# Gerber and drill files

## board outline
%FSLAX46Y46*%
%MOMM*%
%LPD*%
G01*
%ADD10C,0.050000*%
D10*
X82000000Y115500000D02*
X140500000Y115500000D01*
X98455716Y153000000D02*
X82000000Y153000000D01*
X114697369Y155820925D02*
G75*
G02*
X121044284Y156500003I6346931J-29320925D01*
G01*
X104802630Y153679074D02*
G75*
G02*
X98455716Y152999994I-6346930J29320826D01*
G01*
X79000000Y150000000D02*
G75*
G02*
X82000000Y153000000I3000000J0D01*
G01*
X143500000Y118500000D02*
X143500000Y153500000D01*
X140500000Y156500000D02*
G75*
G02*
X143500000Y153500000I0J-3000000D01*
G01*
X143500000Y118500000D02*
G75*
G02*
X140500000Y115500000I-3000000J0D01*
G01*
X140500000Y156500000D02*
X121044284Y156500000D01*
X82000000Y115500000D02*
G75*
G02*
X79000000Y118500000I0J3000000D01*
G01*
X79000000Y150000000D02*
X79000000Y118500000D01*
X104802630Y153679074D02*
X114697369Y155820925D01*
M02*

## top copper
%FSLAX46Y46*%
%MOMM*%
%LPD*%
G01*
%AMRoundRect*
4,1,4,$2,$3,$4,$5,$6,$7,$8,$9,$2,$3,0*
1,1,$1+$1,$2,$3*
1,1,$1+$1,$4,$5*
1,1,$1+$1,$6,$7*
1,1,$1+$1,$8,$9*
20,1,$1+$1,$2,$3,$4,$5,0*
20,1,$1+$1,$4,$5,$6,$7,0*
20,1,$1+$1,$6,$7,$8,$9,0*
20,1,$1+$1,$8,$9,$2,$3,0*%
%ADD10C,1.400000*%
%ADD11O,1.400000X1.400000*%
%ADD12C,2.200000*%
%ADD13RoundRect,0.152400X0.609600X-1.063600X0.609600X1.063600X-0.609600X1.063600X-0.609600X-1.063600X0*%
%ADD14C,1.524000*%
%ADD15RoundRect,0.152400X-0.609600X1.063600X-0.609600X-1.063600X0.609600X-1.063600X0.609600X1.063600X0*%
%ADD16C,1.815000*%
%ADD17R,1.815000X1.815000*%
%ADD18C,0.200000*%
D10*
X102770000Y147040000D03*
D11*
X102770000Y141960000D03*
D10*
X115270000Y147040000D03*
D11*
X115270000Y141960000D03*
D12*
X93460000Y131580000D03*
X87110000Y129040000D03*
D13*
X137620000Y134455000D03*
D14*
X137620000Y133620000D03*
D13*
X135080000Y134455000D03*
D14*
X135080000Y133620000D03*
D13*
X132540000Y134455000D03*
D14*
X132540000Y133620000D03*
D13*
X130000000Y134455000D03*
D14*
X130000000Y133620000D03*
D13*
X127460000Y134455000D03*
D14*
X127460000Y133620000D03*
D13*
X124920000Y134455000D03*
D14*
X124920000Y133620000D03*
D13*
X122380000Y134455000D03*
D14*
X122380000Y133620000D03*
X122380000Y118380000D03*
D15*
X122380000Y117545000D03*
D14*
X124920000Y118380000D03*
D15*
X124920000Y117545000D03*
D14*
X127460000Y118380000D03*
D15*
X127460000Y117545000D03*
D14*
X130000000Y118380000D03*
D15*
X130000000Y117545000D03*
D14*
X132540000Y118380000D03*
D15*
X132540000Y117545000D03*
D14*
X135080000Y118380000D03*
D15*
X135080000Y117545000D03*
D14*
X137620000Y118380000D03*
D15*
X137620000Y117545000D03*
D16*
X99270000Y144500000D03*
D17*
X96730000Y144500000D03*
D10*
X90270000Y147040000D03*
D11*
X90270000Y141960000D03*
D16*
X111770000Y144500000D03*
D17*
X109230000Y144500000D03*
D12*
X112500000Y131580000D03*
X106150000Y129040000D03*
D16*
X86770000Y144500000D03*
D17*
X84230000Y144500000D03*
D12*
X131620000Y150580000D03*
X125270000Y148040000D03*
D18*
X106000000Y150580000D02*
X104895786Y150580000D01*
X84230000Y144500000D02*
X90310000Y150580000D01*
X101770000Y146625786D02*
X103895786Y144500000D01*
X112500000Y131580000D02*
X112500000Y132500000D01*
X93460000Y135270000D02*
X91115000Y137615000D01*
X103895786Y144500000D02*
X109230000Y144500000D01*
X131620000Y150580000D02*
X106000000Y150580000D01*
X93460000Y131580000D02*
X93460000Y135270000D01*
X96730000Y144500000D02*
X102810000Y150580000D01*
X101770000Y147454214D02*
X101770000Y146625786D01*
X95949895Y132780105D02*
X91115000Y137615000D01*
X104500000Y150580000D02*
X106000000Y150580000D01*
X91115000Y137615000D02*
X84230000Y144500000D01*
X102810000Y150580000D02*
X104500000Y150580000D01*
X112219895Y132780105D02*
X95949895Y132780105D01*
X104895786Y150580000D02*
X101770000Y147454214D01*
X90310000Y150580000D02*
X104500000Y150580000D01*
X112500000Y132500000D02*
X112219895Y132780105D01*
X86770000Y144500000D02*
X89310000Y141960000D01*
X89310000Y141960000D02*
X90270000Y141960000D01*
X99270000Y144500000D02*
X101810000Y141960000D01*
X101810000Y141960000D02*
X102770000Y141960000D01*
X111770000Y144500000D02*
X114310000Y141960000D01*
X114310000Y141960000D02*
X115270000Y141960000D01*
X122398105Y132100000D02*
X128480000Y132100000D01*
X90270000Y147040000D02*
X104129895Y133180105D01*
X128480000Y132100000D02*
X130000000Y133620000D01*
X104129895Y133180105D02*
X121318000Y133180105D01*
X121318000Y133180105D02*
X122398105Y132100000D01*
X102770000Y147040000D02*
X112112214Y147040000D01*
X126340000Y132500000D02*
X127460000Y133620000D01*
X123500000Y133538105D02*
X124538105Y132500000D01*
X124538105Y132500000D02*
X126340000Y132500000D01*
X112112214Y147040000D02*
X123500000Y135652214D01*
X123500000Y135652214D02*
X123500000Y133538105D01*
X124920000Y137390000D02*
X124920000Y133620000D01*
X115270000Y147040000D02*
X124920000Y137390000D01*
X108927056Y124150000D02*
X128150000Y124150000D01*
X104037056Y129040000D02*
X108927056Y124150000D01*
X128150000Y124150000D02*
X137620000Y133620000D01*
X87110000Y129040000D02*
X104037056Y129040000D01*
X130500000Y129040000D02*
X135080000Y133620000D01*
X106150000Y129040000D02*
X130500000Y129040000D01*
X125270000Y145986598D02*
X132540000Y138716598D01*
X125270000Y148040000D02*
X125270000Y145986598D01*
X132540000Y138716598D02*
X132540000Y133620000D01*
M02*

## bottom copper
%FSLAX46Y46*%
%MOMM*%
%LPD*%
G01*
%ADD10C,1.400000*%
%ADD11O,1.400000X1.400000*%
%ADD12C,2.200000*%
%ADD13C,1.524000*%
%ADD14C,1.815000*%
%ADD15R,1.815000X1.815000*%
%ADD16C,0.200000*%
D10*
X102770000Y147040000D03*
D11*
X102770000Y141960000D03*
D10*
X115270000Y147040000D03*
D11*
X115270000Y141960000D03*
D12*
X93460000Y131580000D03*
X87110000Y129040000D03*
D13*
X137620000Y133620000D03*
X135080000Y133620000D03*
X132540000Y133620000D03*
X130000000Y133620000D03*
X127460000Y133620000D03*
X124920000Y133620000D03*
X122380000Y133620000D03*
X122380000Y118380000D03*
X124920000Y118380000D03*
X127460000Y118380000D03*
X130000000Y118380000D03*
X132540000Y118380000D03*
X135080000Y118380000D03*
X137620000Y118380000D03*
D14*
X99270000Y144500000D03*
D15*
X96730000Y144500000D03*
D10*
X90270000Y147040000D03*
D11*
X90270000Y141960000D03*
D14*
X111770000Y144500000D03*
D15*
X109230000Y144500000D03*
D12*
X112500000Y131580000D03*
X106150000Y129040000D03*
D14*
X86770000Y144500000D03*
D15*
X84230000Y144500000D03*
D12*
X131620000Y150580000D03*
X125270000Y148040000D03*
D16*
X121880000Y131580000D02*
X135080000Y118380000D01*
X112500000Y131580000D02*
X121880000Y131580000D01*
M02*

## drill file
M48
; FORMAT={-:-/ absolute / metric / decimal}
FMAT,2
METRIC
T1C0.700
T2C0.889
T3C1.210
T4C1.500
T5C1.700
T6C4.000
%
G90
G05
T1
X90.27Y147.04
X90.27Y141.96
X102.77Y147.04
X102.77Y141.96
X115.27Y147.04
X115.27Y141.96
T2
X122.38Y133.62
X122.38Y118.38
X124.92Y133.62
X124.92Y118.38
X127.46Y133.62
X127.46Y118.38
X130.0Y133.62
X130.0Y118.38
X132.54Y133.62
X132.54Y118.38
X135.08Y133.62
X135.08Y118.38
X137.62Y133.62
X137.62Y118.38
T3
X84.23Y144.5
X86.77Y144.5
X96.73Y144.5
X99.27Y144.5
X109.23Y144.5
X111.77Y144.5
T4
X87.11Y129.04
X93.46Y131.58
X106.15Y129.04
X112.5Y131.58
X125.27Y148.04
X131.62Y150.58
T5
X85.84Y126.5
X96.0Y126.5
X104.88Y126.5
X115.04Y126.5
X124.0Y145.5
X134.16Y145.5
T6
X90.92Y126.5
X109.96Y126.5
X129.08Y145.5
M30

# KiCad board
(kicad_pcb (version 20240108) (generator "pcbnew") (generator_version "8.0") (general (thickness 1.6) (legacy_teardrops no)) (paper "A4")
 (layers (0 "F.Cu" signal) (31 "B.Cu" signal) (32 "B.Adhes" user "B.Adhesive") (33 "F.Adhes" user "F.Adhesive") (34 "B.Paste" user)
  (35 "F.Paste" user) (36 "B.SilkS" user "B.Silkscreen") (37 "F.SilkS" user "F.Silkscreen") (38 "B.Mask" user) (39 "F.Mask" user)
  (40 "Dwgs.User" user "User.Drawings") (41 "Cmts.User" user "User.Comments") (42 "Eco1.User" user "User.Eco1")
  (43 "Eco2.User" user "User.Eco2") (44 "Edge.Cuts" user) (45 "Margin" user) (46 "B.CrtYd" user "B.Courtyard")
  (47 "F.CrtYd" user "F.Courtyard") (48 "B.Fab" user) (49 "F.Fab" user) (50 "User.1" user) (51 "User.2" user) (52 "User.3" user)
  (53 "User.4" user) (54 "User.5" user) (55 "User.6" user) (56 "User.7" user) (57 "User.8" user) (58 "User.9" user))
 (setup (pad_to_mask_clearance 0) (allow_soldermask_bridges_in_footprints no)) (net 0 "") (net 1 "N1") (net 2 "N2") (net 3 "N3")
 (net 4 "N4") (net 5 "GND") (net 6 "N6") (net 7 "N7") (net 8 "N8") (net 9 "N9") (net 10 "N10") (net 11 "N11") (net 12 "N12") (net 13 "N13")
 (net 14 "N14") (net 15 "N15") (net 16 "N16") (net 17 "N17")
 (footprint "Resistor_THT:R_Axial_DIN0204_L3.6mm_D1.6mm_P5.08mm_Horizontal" (layer "F.Cu") (at 102.77 -147.04 -90)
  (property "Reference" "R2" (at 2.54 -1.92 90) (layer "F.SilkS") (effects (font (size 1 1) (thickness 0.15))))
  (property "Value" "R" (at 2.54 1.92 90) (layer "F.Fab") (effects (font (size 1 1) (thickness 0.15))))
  (pad "1" thru_hole circle (at 0 0 270) (size 1.4 1.4) (drill 0.7) (layers "*.Cu" "*.Mask") (remove_unused_layers no) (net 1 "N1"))
  (pad "2" thru_hole oval (at 5.08 0 270) (size 1.4 1.4) (drill 0.7) (layers "*.Cu" "*.Mask") (remove_unused_layers no) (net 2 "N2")))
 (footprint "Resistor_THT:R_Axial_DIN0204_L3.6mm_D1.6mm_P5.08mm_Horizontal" (layer "F.Cu") (at 115.27 -147.04 -90)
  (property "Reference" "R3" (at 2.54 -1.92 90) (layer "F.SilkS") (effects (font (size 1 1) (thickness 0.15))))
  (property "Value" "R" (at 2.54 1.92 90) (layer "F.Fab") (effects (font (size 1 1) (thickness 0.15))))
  (pad "1" thru_hole circle (at 0 0 270) (size 1.4 1.4) (drill 0.7) (layers "*.Cu" "*.Mask") (remove_unused_layers no) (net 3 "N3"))
  (pad "2" thru_hole oval (at 5.08 0 270) (size 1.4 1.4) (drill 0.7) (layers "*.Cu" "*.Mask") (remove_unused_layers no) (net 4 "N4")))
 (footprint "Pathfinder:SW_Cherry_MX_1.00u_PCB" (layer "F.Cu") (at 93.46 -131.58)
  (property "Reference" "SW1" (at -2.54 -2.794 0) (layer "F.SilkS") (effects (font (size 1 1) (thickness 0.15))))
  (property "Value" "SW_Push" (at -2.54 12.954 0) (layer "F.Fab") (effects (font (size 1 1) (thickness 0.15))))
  (pad "" np_thru_hole circle (at -7.62 5.08) (size 1.7 1.7) (drill 1.7) (layers "*.Cu" "*.Mask"))
  (pad "" np_thru_hole circle (at -2.54 5.08) (size 4 4) (drill 4) (layers "*.Cu" "*.Mask"))
  (pad "" np_thru_hole circle (at 2.54 5.08) (size 1.7 1.7) (drill 1.7) (layers "*.Cu" "*.Mask"))
  (pad "1" thru_hole circle (at 0 0) (size 2.2 2.2) (drill 1.5) (layers "*.Cu" "*.Mask") (remove_unused_layers no) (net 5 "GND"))
  (pad "2" thru_hole circle (at -6.35 2.54) (size 2.2 2.2) (drill 1.5) (layers "*.Cu" "*.Mask") (remove_unused_layers no) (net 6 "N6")))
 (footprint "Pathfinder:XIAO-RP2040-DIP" (layer "F.Cu") (at 130 -126 -90)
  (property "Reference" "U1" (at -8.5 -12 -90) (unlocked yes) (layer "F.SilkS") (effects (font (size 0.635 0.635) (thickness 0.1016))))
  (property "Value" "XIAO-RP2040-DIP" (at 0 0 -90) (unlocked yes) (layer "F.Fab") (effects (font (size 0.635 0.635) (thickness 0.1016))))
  (pad "1" smd roundrect (at -8.455 -7.62 90) (size 2.432 1.524) (layers "F.Cu" "F.Mask") (roundrect_rratio 0.1) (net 6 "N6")
   (thermal_bridge_angle 45))
  (pad "1" thru_hole circle (at -7.62 -7.62 90) (size 1.524 1.524) (drill 0.889) (layers "*.Cu" "*.Mask") (remove_unused_layers no)
   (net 6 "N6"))
  (pad "2" smd roundrect (at -8.455 -5.08 90) (size 2.432 1.524) (layers "F.Cu" "F.Mask") (roundrect_rratio 0.1) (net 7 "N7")
   (thermal_bridge_angle 45))
  (pad "2" thru_hole circle (at -7.62 -5.08 90) (size 1.524 1.524) (drill 0.889) (layers "*.Cu" "*.Mask") (remove_unused_layers no)
   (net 7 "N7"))
  (pad "3" smd roundrect (at -8.455 -2.54 90) (size 2.432 1.524) (layers "F.Cu" "F.Mask") (roundrect_rratio 0.1) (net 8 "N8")
   (thermal_bridge_angle 45))
  (pad "3" thru_hole circle (at -7.62 -2.54 90) (size 1.524 1.524) (drill 0.889) (layers "*.Cu" "*.Mask") (remove_unused_layers no)
   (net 8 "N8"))
  (pad "4" smd roundrect (at -8.455 0 90) (size 2.432 1.524) (layers "F.Cu" "F.Mask") (roundrect_rratio 0.1) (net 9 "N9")
   (thermal_bridge_angle 45))
  (pad "4" thru_hole circle (at -7.62 0 90) (size 1.524 1.524) (drill 0.889) (layers "*.Cu" "*.Mask") (remove_unused_layers no) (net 9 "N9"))
  (pad "5" smd roundrect (at -8.455 2.54 90) (size 2.432 1.524) (layers "F.Cu" "F.Mask") (roundrect_rratio 0.1) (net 1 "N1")
   (thermal_bridge_angle 45))
  (pad "5" thru_hole circle (at -7.62 2.54 90) (size 1.524 1.524) (drill 0.889) (layers "*.Cu" "*.Mask") (remove_unused_layers no)
   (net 1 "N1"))
  (pad "6" smd roundrect (at -8.455 5.08 90) (size 2.432 1.524) (layers "F.Cu" "F.Mask") (roundrect_rratio 0.1) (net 3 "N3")
   (thermal_bridge_angle 45))
  (pad "6" thru_hole circle (at -7.62 5.08 90) (size 1.524 1.524) (drill 0.889) (layers "*.Cu" "*.Mask") (remove_unused_layers no)
   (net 3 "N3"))
  (pad "7" smd roundrect (at -8.455 7.62 90) (size 2.432 1.524) (layers "F.Cu" "F.Mask") (roundrect_rratio 0.1) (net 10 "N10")
   (thermal_bridge_angle 45))
  (pad "7" thru_hole circle (at -7.62 7.62 90) (size 1.524 1.524) (drill 0.889) (layers "*.Cu" "*.Mask") (remove_unused_layers no)
   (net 10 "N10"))
  (pad "8" thru_hole circle (at 7.62 7.62 270) (size 1.524 1.524) (drill 0.889) (layers "*.Cu" "*.Mask") (remove_unused_layers no)
   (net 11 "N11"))
  (pad "8" smd roundrect (at 8.455 7.62 270) (size 2.432 1.524) (layers "F.Cu" "F.Mask") (roundrect_rratio 0.1) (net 11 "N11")
   (thermal_bridge_angle 45))
  (pad "9" thru_hole circle (at 7.62 5.08 270) (size 1.524 1.524) (drill 0.889) (layers "*.Cu" "*.Mask") (remove_unused_layers no)
   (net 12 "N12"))
  (pad "9" smd roundrect (at 8.455 5.08 270) (size 2.432 1.524) (layers "F.Cu" "F.Mask") (roundrect_rratio 0.1) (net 12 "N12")
   (thermal_bridge_angle 45))
  (pad "10" thru_hole circle (at 7.62 2.54 270) (size 1.524 1.524) (drill 0.889) (layers "*.Cu" "*.Mask") (remove_unused_layers no)
   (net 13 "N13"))
  (pad "10" smd roundrect (at 8.455 2.54 270) (size 2.432 1.524) (layers "F.Cu" "F.Mask") (roundrect_rratio 0.1) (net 13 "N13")
   (thermal_bridge_angle 45))
  (pad "11" thru_hole circle (at 7.62 0 270) (size 1.524 1.524) (drill 0.889) (layers "*.Cu" "*.Mask") (remove_unused_layers no)
   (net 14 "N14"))
  (pad "11" smd roundrect (at 8.455 0 270) (size 2.432 1.524) (layers "F.Cu" "F.Mask") (roundrect_rratio 0.1) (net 14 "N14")
   (thermal_bridge_angle 45))
  (pad "12" thru_hole circle (at 7.62 -2.54 270) (size 1.524 1.524) (drill 0.889) (layers "*.Cu" "*.Mask") (remove_unused_layers no)
   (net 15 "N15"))
  (pad "12" smd roundrect (at 8.455 -2.54 270) (size 2.432 1.524) (layers "F.Cu" "F.Mask") (roundrect_rratio 0.1) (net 15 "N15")
   (thermal_bridge_angle 45))
  (pad "13" thru_hole circle (at 7.62 -5.08 270) (size 1.524 1.524) (drill 0.889) (layers "*.Cu" "*.Mask") (remove_unused_layers no)
   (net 5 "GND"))
  (pad "13" smd roundrect (at 8.455 -5.08 270) (size 2.432 1.524) (layers "F.Cu" "F.Mask") (roundrect_rratio 0.1) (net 5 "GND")
   (thermal_bridge_angle 45))
  (pad "14" thru_hole circle (at 7.62 -7.62 270) (size 1.524 1.524) (drill 0.889) (layers "*.Cu" "*.Mask") (remove_unused_layers no)
   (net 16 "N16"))
  (pad "14" smd roundrect (at 8.455 -7.62 270) (size 2.432 1.524) (layers "F.Cu" "F.Mask") (roundrect_rratio 0.1) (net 16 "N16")
   (thermal_bridge_angle 45)))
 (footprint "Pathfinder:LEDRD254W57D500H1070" (layer "F.Cu") (at 98 -144.5)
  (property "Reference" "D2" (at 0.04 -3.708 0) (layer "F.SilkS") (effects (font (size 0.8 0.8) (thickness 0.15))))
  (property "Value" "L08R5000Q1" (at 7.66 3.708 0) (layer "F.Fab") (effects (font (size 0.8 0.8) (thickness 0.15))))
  (pad "A" thru_hole circle (at 1.27 0) (size 1.815 1.815) (drill 1.21) (layers "*.Cu" "*.Mask") (remove_unused_layers no) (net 2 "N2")
   (solder_mask_margin 0.102))
  (pad "C" thru_hole rect (at -1.27 0) (size 1.815 1.815) (drill 1.21) (layers "*.Cu" "*.Mask") (remove_unused_layers no) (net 5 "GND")
   (solder_mask_margin 0.102)))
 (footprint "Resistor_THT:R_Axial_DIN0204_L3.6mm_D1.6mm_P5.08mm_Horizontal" (layer "F.Cu") (at 90.27 -147.04 -90)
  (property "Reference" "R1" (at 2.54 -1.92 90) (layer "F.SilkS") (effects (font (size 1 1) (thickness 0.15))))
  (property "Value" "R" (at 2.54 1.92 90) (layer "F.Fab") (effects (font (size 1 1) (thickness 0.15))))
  (pad "1" thru_hole circle (at 0 0 270) (size 1.4 1.4) (drill 0.7) (layers "*.Cu" "*.Mask") (remove_unused_layers no) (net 9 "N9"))
  (pad "2" thru_hole oval (at 5.08 0 270) (size 1.4 1.4) (drill 0.7) (layers "*.Cu" "*.Mask") (remove_unused_layers no) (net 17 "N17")))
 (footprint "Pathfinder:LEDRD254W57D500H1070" (layer "F.Cu") (at 110.5 -144.5)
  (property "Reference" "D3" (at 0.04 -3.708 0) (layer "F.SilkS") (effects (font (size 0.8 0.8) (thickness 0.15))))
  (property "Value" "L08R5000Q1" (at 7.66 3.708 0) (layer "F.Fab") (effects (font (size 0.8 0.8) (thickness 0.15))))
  (pad "A" thru_hole circle (at 1.27 0) (size 1.815 1.815) (drill 1.21) (layers "*.Cu" "*.Mask") (remove_unused_layers no) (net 4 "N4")
   (solder_mask_margin 0.102))
  (pad "C" thru_hole rect (at -1.27 0) (size 1.815 1.815) (drill 1.21) (layers "*.Cu" "*.Mask") (remove_unused_layers no) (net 5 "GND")
   (solder_mask_margin 0.102)))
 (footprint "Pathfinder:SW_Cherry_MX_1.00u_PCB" (layer "F.Cu") (at 112.5 -131.58)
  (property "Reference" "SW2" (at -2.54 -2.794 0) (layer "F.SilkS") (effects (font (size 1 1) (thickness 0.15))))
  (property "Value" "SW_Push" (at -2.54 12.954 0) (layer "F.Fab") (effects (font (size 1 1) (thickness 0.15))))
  (pad "" np_thru_hole circle (at -7.62 5.08) (size 1.7 1.7) (drill 1.7) (layers "*.Cu" "*.Mask"))
  (pad "" np_thru_hole circle (at -2.54 5.08) (size 4 4) (drill 4) (layers "*.Cu" "*.Mask"))
  (pad "" np_thru_hole circle (at 2.54 5.08) (size 1.7 1.7) (drill 1.7) (layers "*.Cu" "*.Mask"))
  (pad "1" thru_hole circle (at 0 0) (size 2.2 2.2) (drill 1.5) (layers "*.Cu" "*.Mask") (remove_unused_layers no) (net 5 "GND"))
  (pad "2" thru_hole circle (at -6.35 2.54) (size 2.2 2.2) (drill 1.5) (layers "*.Cu" "*.Mask") (remove_unused_layers no) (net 7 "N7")))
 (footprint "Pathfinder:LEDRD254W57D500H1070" (layer "F.Cu") (at 85.5 -144.5)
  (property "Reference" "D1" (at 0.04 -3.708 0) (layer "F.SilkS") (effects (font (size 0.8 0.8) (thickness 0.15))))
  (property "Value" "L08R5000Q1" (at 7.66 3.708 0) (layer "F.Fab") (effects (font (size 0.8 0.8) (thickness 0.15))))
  (pad "A" thru_hole circle (at 1.27 0) (size 1.815 1.815) (drill 1.21) (layers "*.Cu" "*.Mask") (remove_unused_layers no) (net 17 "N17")
   (solder_mask_margin 0.102))
  (pad "C" thru_hole rect (at -1.27 0) (size 1.815 1.815) (drill 1.21) (layers "*.Cu" "*.Mask") (remove_unused_layers no) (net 5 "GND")
   (solder_mask_margin 0.102)))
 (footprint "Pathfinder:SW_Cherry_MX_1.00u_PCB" (layer "F.Cu") (at 131.62 -150.58)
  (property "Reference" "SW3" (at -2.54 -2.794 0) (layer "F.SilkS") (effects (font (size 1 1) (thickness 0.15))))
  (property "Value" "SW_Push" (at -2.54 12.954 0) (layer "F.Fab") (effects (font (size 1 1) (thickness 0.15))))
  (pad "" np_thru_hole circle (at -7.62 5.08) (size 1.7 1.7) (drill 1.7) (layers "*.Cu" "*.Mask"))
  (pad "" np_thru_hole circle (at -2.54 5.08) (size 4 4) (drill 4) (layers "*.Cu" "*.Mask"))
  (pad "" np_thru_hole circle (at 2.54 5.08) (size 1.7 1.7) (drill 1.7) (layers "*.Cu" "*.Mask"))
  (pad "1" thru_hole circle (at 0 0) (size 2.2 2.2) (drill 1.5) (layers "*.Cu" "*.Mask") (remove_unused_layers no) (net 5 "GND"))
  (pad "2" thru_hole circle (at -6.35 2.54) (size 2.2 2.2) (drill 1.5) (layers "*.Cu" "*.Mask") (remove_unused_layers no) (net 8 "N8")))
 (gr_line (start 82 -115.5) (end 140.5 -115.5) (stroke (width 0.05) (type default)) (layer "Edge.Cuts"))
 (gr_line (start 98.455716 -153) (end 82 -153) (stroke (width 0.05) (type default)) (layer "Edge.Cuts"))
 (gr_arc (start 114.697369 -155.820925) (mid 117.852714 -156.329748) (end 121.044284 -156.5) (stroke (width 0.05) (type default))
  (layer "Edge.Cuts"))
 (gr_arc (start 104.80263 -153.679074) (mid 101.647285 -153.170251) (end 98.455716 -153) (stroke (width 0.05) (type default))
  (layer "Edge.Cuts"))
 (gr_arc (start 79 -150) (mid 79.87868 -152.12132) (end 82 -153) (stroke (width 0.05) (type default)) (layer "Edge.Cuts"))
 (gr_line (start 143.5 -118.5) (end 143.5 -153.5) (stroke (width 0.05) (type default)) (layer "Edge.Cuts"))
 (gr_arc (start 140.5 -156.5) (mid 142.62132 -155.62132) (end 143.5 -153.5) (stroke (width 0.05) (type default)) (layer "Edge.Cuts"))
 (gr_arc (start 143.5 -118.5) (mid 142.62132 -116.37868) (end 140.5 -115.5) (stroke (width 0.05) (type default)) (layer "Edge.Cuts"))
 (gr_line (start 140.5 -156.5) (end 121.044284 -156.5) (stroke (width 0.05) (type default)) (layer "Edge.Cuts"))
 (gr_arc (start 82 -115.5) (mid 79.87868 -116.37868) (end 79 -118.5) (stroke (width 0.05) (type default)) (layer "Edge.Cuts"))
 (gr_line (start 79 -150) (end 79 -118.5) (stroke (width 0.05) (type default)) (layer "Edge.Cuts"))
 (gr_line (start 104.80263 -153.679074) (end 114.697369 -155.820925) (stroke (width 0.05) (type default)) (layer "Edge.Cuts"))
 (segment (start 106 -150.58) (end 104.895786 -150.58) (width 0.2) (layer "F.Cu") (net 5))
 (segment (start 84.23 -144.5) (end 90.31 -150.58) (width 0.2) (layer "F.Cu") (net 5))
 (segment (start 101.77 -146.625786) (end 103.895786 -144.5) (width 0.2) (layer "F.Cu") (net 5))
 (segment (start 112.5 -131.58) (end 112.5 -132.5) (width 0.2) (layer "F.Cu") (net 5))
 (segment (start 93.46 -135.27) (end 91.115 -137.615) (width 0.2) (layer "F.Cu") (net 5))
 (segment (start 103.895786 -144.5) (end 109.23 -144.5) (width 0.2) (layer "F.Cu") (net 5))
 (segment (start 131.62 -150.58) (end 106 -150.58) (width 0.2) (layer "F.Cu") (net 5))
 (segment (start 93.46 -131.58) (end 93.46 -135.27) (width 0.2) (layer "F.Cu") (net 5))
 (segment (start 96.73 -144.5) (end 102.81 -150.58) (width 0.2) (layer "F.Cu") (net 5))
 (segment (start 101.77 -147.454214) (end 101.77 -146.625786) (width 0.2) (layer "F.Cu") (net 5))
 (segment (start 95.949895 -132.780105) (end 91.115 -137.615) (width 0.2) (layer "F.Cu") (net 5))
 (segment (start 104.5 -150.58) (end 106 -150.58) (width 0.2) (layer "F.Cu") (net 5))
 (segment (start 91.115 -137.615) (end 84.23 -144.5) (width 0.2) (layer "F.Cu") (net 5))
 (segment (start 102.81 -150.58) (end 104.5 -150.58) (width 0.2) (layer "F.Cu") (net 5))
 (segment (start 112.219895 -132.780105) (end 95.949895 -132.780105) (width 0.2) (layer "F.Cu") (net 5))
 (segment (start 104.895786 -150.58) (end 101.77 -147.454214) (width 0.2) (layer "F.Cu") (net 5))
 (segment (start 90.31 -150.58) (end 104.5 -150.58) (width 0.2) (layer "F.Cu") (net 5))
 (segment (start 112.5 -132.5) (end 112.219895 -132.780105) (width 0.2) (layer "F.Cu") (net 5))
 (segment (start 121.88 -131.58) (end 135.08 -118.38) (width 0.2) (layer "B.Cu") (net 5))
 (segment (start 112.5 -131.58) (end 121.88 -131.58) (width 0.2) (layer "B.Cu") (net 5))
 (segment (start 86.77 -144.5) (end 89.31 -141.96) (width 0.2) (layer "F.Cu") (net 17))
 (segment (start 89.31 -141.96) (end 90.27 -141.96) (width 0.2) (layer "F.Cu") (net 17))
 (segment (start 99.27 -144.5) (end 101.81 -141.96) (width 0.2) (layer "F.Cu") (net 2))
 (segment (start 101.81 -141.96) (end 102.77 -141.96) (width 0.2) (layer "F.Cu") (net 2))
 (segment (start 111.77 -144.5) (end 114.31 -141.96) (width 0.2) (layer "F.Cu") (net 4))
 (segment (start 114.31 -141.96) (end 115.27 -141.96) (width 0.2) (layer "F.Cu") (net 4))
 (segment (start 122.398105 -132.1) (end 128.48 -132.1) (width 0.2) (layer "F.Cu") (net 9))
 (segment (start 90.27 -147.04) (end 104.129895 -133.180105) (width 0.2) (layer "F.Cu") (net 9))
 (segment (start 128.48 -132.1) (end 130 -133.62) (width 0.2) (layer "F.Cu") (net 9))
 (segment (start 104.129895 -133.180105) (end 121.318 -133.180105) (width 0.2) (layer "F.Cu") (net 9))
 (segment (start 121.318 -133.180105) (end 122.398105 -132.1) (width 0.2) (layer "F.Cu") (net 9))
 (segment (start 102.77 -147.04) (end 112.112214 -147.04) (width 0.2) (layer "F.Cu") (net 1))
 (segment (start 126.34 -132.5) (end 127.46 -133.62) (width 0.2) (layer "F.Cu") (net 1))
 (segment (start 123.5 -133.538105) (end 124.538105 -132.5) (width 0.2) (layer "F.Cu") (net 1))
 (segment (start 124.538105 -132.5) (end 126.34 -132.5) (width 0.2) (layer "F.Cu") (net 1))
 (segment (start 112.112214 -147.04) (end 123.5 -135.652214) (width 0.2) (layer "F.Cu") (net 1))
 (segment (start 123.5 -135.652214) (end 123.5 -133.538105) (width 0.2) (layer "F.Cu") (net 1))
 (segment (start 124.92 -137.39) (end 124.92 -133.62) (width 0.2) (layer "F.Cu") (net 3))
 (segment (start 115.27 -147.04) (end 124.92 -137.39) (width 0.2) (layer "F.Cu") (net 3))
 (segment (start 108.927056 -124.15) (end 128.15 -124.15) (width 0.2) (layer "F.Cu") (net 6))
 (segment (start 104.037056 -129.04) (end 108.927056 -124.15) (width 0.2) (layer "F.Cu") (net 6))
 (segment (start 128.15 -124.15) (end 137.62 -133.62) (width 0.2) (layer "F.Cu") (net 6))
 (segment (start 87.11 -129.04) (end 104.037056 -129.04) (width 0.2) (layer "F.Cu") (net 6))
 (segment (start 130.5 -129.04) (end 135.08 -133.62) (width 0.2) (layer "F.Cu") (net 7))
 (segment (start 106.15 -129.04) (end 130.5 -129.04) (width 0.2) (layer "F.Cu") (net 7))
 (segment (start 125.27 -145.986598) (end 132.54 -138.716598) (width 0.2) (layer "F.Cu") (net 8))
 (segment (start 125.27 -148.04) (end 125.27 -145.986598) (width 0.2) (layer "F.Cu") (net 8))
 (segment (start 132.54 -138.716598) (end 132.54 -133.62) (width 0.2) (layer "F.Cu") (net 8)))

